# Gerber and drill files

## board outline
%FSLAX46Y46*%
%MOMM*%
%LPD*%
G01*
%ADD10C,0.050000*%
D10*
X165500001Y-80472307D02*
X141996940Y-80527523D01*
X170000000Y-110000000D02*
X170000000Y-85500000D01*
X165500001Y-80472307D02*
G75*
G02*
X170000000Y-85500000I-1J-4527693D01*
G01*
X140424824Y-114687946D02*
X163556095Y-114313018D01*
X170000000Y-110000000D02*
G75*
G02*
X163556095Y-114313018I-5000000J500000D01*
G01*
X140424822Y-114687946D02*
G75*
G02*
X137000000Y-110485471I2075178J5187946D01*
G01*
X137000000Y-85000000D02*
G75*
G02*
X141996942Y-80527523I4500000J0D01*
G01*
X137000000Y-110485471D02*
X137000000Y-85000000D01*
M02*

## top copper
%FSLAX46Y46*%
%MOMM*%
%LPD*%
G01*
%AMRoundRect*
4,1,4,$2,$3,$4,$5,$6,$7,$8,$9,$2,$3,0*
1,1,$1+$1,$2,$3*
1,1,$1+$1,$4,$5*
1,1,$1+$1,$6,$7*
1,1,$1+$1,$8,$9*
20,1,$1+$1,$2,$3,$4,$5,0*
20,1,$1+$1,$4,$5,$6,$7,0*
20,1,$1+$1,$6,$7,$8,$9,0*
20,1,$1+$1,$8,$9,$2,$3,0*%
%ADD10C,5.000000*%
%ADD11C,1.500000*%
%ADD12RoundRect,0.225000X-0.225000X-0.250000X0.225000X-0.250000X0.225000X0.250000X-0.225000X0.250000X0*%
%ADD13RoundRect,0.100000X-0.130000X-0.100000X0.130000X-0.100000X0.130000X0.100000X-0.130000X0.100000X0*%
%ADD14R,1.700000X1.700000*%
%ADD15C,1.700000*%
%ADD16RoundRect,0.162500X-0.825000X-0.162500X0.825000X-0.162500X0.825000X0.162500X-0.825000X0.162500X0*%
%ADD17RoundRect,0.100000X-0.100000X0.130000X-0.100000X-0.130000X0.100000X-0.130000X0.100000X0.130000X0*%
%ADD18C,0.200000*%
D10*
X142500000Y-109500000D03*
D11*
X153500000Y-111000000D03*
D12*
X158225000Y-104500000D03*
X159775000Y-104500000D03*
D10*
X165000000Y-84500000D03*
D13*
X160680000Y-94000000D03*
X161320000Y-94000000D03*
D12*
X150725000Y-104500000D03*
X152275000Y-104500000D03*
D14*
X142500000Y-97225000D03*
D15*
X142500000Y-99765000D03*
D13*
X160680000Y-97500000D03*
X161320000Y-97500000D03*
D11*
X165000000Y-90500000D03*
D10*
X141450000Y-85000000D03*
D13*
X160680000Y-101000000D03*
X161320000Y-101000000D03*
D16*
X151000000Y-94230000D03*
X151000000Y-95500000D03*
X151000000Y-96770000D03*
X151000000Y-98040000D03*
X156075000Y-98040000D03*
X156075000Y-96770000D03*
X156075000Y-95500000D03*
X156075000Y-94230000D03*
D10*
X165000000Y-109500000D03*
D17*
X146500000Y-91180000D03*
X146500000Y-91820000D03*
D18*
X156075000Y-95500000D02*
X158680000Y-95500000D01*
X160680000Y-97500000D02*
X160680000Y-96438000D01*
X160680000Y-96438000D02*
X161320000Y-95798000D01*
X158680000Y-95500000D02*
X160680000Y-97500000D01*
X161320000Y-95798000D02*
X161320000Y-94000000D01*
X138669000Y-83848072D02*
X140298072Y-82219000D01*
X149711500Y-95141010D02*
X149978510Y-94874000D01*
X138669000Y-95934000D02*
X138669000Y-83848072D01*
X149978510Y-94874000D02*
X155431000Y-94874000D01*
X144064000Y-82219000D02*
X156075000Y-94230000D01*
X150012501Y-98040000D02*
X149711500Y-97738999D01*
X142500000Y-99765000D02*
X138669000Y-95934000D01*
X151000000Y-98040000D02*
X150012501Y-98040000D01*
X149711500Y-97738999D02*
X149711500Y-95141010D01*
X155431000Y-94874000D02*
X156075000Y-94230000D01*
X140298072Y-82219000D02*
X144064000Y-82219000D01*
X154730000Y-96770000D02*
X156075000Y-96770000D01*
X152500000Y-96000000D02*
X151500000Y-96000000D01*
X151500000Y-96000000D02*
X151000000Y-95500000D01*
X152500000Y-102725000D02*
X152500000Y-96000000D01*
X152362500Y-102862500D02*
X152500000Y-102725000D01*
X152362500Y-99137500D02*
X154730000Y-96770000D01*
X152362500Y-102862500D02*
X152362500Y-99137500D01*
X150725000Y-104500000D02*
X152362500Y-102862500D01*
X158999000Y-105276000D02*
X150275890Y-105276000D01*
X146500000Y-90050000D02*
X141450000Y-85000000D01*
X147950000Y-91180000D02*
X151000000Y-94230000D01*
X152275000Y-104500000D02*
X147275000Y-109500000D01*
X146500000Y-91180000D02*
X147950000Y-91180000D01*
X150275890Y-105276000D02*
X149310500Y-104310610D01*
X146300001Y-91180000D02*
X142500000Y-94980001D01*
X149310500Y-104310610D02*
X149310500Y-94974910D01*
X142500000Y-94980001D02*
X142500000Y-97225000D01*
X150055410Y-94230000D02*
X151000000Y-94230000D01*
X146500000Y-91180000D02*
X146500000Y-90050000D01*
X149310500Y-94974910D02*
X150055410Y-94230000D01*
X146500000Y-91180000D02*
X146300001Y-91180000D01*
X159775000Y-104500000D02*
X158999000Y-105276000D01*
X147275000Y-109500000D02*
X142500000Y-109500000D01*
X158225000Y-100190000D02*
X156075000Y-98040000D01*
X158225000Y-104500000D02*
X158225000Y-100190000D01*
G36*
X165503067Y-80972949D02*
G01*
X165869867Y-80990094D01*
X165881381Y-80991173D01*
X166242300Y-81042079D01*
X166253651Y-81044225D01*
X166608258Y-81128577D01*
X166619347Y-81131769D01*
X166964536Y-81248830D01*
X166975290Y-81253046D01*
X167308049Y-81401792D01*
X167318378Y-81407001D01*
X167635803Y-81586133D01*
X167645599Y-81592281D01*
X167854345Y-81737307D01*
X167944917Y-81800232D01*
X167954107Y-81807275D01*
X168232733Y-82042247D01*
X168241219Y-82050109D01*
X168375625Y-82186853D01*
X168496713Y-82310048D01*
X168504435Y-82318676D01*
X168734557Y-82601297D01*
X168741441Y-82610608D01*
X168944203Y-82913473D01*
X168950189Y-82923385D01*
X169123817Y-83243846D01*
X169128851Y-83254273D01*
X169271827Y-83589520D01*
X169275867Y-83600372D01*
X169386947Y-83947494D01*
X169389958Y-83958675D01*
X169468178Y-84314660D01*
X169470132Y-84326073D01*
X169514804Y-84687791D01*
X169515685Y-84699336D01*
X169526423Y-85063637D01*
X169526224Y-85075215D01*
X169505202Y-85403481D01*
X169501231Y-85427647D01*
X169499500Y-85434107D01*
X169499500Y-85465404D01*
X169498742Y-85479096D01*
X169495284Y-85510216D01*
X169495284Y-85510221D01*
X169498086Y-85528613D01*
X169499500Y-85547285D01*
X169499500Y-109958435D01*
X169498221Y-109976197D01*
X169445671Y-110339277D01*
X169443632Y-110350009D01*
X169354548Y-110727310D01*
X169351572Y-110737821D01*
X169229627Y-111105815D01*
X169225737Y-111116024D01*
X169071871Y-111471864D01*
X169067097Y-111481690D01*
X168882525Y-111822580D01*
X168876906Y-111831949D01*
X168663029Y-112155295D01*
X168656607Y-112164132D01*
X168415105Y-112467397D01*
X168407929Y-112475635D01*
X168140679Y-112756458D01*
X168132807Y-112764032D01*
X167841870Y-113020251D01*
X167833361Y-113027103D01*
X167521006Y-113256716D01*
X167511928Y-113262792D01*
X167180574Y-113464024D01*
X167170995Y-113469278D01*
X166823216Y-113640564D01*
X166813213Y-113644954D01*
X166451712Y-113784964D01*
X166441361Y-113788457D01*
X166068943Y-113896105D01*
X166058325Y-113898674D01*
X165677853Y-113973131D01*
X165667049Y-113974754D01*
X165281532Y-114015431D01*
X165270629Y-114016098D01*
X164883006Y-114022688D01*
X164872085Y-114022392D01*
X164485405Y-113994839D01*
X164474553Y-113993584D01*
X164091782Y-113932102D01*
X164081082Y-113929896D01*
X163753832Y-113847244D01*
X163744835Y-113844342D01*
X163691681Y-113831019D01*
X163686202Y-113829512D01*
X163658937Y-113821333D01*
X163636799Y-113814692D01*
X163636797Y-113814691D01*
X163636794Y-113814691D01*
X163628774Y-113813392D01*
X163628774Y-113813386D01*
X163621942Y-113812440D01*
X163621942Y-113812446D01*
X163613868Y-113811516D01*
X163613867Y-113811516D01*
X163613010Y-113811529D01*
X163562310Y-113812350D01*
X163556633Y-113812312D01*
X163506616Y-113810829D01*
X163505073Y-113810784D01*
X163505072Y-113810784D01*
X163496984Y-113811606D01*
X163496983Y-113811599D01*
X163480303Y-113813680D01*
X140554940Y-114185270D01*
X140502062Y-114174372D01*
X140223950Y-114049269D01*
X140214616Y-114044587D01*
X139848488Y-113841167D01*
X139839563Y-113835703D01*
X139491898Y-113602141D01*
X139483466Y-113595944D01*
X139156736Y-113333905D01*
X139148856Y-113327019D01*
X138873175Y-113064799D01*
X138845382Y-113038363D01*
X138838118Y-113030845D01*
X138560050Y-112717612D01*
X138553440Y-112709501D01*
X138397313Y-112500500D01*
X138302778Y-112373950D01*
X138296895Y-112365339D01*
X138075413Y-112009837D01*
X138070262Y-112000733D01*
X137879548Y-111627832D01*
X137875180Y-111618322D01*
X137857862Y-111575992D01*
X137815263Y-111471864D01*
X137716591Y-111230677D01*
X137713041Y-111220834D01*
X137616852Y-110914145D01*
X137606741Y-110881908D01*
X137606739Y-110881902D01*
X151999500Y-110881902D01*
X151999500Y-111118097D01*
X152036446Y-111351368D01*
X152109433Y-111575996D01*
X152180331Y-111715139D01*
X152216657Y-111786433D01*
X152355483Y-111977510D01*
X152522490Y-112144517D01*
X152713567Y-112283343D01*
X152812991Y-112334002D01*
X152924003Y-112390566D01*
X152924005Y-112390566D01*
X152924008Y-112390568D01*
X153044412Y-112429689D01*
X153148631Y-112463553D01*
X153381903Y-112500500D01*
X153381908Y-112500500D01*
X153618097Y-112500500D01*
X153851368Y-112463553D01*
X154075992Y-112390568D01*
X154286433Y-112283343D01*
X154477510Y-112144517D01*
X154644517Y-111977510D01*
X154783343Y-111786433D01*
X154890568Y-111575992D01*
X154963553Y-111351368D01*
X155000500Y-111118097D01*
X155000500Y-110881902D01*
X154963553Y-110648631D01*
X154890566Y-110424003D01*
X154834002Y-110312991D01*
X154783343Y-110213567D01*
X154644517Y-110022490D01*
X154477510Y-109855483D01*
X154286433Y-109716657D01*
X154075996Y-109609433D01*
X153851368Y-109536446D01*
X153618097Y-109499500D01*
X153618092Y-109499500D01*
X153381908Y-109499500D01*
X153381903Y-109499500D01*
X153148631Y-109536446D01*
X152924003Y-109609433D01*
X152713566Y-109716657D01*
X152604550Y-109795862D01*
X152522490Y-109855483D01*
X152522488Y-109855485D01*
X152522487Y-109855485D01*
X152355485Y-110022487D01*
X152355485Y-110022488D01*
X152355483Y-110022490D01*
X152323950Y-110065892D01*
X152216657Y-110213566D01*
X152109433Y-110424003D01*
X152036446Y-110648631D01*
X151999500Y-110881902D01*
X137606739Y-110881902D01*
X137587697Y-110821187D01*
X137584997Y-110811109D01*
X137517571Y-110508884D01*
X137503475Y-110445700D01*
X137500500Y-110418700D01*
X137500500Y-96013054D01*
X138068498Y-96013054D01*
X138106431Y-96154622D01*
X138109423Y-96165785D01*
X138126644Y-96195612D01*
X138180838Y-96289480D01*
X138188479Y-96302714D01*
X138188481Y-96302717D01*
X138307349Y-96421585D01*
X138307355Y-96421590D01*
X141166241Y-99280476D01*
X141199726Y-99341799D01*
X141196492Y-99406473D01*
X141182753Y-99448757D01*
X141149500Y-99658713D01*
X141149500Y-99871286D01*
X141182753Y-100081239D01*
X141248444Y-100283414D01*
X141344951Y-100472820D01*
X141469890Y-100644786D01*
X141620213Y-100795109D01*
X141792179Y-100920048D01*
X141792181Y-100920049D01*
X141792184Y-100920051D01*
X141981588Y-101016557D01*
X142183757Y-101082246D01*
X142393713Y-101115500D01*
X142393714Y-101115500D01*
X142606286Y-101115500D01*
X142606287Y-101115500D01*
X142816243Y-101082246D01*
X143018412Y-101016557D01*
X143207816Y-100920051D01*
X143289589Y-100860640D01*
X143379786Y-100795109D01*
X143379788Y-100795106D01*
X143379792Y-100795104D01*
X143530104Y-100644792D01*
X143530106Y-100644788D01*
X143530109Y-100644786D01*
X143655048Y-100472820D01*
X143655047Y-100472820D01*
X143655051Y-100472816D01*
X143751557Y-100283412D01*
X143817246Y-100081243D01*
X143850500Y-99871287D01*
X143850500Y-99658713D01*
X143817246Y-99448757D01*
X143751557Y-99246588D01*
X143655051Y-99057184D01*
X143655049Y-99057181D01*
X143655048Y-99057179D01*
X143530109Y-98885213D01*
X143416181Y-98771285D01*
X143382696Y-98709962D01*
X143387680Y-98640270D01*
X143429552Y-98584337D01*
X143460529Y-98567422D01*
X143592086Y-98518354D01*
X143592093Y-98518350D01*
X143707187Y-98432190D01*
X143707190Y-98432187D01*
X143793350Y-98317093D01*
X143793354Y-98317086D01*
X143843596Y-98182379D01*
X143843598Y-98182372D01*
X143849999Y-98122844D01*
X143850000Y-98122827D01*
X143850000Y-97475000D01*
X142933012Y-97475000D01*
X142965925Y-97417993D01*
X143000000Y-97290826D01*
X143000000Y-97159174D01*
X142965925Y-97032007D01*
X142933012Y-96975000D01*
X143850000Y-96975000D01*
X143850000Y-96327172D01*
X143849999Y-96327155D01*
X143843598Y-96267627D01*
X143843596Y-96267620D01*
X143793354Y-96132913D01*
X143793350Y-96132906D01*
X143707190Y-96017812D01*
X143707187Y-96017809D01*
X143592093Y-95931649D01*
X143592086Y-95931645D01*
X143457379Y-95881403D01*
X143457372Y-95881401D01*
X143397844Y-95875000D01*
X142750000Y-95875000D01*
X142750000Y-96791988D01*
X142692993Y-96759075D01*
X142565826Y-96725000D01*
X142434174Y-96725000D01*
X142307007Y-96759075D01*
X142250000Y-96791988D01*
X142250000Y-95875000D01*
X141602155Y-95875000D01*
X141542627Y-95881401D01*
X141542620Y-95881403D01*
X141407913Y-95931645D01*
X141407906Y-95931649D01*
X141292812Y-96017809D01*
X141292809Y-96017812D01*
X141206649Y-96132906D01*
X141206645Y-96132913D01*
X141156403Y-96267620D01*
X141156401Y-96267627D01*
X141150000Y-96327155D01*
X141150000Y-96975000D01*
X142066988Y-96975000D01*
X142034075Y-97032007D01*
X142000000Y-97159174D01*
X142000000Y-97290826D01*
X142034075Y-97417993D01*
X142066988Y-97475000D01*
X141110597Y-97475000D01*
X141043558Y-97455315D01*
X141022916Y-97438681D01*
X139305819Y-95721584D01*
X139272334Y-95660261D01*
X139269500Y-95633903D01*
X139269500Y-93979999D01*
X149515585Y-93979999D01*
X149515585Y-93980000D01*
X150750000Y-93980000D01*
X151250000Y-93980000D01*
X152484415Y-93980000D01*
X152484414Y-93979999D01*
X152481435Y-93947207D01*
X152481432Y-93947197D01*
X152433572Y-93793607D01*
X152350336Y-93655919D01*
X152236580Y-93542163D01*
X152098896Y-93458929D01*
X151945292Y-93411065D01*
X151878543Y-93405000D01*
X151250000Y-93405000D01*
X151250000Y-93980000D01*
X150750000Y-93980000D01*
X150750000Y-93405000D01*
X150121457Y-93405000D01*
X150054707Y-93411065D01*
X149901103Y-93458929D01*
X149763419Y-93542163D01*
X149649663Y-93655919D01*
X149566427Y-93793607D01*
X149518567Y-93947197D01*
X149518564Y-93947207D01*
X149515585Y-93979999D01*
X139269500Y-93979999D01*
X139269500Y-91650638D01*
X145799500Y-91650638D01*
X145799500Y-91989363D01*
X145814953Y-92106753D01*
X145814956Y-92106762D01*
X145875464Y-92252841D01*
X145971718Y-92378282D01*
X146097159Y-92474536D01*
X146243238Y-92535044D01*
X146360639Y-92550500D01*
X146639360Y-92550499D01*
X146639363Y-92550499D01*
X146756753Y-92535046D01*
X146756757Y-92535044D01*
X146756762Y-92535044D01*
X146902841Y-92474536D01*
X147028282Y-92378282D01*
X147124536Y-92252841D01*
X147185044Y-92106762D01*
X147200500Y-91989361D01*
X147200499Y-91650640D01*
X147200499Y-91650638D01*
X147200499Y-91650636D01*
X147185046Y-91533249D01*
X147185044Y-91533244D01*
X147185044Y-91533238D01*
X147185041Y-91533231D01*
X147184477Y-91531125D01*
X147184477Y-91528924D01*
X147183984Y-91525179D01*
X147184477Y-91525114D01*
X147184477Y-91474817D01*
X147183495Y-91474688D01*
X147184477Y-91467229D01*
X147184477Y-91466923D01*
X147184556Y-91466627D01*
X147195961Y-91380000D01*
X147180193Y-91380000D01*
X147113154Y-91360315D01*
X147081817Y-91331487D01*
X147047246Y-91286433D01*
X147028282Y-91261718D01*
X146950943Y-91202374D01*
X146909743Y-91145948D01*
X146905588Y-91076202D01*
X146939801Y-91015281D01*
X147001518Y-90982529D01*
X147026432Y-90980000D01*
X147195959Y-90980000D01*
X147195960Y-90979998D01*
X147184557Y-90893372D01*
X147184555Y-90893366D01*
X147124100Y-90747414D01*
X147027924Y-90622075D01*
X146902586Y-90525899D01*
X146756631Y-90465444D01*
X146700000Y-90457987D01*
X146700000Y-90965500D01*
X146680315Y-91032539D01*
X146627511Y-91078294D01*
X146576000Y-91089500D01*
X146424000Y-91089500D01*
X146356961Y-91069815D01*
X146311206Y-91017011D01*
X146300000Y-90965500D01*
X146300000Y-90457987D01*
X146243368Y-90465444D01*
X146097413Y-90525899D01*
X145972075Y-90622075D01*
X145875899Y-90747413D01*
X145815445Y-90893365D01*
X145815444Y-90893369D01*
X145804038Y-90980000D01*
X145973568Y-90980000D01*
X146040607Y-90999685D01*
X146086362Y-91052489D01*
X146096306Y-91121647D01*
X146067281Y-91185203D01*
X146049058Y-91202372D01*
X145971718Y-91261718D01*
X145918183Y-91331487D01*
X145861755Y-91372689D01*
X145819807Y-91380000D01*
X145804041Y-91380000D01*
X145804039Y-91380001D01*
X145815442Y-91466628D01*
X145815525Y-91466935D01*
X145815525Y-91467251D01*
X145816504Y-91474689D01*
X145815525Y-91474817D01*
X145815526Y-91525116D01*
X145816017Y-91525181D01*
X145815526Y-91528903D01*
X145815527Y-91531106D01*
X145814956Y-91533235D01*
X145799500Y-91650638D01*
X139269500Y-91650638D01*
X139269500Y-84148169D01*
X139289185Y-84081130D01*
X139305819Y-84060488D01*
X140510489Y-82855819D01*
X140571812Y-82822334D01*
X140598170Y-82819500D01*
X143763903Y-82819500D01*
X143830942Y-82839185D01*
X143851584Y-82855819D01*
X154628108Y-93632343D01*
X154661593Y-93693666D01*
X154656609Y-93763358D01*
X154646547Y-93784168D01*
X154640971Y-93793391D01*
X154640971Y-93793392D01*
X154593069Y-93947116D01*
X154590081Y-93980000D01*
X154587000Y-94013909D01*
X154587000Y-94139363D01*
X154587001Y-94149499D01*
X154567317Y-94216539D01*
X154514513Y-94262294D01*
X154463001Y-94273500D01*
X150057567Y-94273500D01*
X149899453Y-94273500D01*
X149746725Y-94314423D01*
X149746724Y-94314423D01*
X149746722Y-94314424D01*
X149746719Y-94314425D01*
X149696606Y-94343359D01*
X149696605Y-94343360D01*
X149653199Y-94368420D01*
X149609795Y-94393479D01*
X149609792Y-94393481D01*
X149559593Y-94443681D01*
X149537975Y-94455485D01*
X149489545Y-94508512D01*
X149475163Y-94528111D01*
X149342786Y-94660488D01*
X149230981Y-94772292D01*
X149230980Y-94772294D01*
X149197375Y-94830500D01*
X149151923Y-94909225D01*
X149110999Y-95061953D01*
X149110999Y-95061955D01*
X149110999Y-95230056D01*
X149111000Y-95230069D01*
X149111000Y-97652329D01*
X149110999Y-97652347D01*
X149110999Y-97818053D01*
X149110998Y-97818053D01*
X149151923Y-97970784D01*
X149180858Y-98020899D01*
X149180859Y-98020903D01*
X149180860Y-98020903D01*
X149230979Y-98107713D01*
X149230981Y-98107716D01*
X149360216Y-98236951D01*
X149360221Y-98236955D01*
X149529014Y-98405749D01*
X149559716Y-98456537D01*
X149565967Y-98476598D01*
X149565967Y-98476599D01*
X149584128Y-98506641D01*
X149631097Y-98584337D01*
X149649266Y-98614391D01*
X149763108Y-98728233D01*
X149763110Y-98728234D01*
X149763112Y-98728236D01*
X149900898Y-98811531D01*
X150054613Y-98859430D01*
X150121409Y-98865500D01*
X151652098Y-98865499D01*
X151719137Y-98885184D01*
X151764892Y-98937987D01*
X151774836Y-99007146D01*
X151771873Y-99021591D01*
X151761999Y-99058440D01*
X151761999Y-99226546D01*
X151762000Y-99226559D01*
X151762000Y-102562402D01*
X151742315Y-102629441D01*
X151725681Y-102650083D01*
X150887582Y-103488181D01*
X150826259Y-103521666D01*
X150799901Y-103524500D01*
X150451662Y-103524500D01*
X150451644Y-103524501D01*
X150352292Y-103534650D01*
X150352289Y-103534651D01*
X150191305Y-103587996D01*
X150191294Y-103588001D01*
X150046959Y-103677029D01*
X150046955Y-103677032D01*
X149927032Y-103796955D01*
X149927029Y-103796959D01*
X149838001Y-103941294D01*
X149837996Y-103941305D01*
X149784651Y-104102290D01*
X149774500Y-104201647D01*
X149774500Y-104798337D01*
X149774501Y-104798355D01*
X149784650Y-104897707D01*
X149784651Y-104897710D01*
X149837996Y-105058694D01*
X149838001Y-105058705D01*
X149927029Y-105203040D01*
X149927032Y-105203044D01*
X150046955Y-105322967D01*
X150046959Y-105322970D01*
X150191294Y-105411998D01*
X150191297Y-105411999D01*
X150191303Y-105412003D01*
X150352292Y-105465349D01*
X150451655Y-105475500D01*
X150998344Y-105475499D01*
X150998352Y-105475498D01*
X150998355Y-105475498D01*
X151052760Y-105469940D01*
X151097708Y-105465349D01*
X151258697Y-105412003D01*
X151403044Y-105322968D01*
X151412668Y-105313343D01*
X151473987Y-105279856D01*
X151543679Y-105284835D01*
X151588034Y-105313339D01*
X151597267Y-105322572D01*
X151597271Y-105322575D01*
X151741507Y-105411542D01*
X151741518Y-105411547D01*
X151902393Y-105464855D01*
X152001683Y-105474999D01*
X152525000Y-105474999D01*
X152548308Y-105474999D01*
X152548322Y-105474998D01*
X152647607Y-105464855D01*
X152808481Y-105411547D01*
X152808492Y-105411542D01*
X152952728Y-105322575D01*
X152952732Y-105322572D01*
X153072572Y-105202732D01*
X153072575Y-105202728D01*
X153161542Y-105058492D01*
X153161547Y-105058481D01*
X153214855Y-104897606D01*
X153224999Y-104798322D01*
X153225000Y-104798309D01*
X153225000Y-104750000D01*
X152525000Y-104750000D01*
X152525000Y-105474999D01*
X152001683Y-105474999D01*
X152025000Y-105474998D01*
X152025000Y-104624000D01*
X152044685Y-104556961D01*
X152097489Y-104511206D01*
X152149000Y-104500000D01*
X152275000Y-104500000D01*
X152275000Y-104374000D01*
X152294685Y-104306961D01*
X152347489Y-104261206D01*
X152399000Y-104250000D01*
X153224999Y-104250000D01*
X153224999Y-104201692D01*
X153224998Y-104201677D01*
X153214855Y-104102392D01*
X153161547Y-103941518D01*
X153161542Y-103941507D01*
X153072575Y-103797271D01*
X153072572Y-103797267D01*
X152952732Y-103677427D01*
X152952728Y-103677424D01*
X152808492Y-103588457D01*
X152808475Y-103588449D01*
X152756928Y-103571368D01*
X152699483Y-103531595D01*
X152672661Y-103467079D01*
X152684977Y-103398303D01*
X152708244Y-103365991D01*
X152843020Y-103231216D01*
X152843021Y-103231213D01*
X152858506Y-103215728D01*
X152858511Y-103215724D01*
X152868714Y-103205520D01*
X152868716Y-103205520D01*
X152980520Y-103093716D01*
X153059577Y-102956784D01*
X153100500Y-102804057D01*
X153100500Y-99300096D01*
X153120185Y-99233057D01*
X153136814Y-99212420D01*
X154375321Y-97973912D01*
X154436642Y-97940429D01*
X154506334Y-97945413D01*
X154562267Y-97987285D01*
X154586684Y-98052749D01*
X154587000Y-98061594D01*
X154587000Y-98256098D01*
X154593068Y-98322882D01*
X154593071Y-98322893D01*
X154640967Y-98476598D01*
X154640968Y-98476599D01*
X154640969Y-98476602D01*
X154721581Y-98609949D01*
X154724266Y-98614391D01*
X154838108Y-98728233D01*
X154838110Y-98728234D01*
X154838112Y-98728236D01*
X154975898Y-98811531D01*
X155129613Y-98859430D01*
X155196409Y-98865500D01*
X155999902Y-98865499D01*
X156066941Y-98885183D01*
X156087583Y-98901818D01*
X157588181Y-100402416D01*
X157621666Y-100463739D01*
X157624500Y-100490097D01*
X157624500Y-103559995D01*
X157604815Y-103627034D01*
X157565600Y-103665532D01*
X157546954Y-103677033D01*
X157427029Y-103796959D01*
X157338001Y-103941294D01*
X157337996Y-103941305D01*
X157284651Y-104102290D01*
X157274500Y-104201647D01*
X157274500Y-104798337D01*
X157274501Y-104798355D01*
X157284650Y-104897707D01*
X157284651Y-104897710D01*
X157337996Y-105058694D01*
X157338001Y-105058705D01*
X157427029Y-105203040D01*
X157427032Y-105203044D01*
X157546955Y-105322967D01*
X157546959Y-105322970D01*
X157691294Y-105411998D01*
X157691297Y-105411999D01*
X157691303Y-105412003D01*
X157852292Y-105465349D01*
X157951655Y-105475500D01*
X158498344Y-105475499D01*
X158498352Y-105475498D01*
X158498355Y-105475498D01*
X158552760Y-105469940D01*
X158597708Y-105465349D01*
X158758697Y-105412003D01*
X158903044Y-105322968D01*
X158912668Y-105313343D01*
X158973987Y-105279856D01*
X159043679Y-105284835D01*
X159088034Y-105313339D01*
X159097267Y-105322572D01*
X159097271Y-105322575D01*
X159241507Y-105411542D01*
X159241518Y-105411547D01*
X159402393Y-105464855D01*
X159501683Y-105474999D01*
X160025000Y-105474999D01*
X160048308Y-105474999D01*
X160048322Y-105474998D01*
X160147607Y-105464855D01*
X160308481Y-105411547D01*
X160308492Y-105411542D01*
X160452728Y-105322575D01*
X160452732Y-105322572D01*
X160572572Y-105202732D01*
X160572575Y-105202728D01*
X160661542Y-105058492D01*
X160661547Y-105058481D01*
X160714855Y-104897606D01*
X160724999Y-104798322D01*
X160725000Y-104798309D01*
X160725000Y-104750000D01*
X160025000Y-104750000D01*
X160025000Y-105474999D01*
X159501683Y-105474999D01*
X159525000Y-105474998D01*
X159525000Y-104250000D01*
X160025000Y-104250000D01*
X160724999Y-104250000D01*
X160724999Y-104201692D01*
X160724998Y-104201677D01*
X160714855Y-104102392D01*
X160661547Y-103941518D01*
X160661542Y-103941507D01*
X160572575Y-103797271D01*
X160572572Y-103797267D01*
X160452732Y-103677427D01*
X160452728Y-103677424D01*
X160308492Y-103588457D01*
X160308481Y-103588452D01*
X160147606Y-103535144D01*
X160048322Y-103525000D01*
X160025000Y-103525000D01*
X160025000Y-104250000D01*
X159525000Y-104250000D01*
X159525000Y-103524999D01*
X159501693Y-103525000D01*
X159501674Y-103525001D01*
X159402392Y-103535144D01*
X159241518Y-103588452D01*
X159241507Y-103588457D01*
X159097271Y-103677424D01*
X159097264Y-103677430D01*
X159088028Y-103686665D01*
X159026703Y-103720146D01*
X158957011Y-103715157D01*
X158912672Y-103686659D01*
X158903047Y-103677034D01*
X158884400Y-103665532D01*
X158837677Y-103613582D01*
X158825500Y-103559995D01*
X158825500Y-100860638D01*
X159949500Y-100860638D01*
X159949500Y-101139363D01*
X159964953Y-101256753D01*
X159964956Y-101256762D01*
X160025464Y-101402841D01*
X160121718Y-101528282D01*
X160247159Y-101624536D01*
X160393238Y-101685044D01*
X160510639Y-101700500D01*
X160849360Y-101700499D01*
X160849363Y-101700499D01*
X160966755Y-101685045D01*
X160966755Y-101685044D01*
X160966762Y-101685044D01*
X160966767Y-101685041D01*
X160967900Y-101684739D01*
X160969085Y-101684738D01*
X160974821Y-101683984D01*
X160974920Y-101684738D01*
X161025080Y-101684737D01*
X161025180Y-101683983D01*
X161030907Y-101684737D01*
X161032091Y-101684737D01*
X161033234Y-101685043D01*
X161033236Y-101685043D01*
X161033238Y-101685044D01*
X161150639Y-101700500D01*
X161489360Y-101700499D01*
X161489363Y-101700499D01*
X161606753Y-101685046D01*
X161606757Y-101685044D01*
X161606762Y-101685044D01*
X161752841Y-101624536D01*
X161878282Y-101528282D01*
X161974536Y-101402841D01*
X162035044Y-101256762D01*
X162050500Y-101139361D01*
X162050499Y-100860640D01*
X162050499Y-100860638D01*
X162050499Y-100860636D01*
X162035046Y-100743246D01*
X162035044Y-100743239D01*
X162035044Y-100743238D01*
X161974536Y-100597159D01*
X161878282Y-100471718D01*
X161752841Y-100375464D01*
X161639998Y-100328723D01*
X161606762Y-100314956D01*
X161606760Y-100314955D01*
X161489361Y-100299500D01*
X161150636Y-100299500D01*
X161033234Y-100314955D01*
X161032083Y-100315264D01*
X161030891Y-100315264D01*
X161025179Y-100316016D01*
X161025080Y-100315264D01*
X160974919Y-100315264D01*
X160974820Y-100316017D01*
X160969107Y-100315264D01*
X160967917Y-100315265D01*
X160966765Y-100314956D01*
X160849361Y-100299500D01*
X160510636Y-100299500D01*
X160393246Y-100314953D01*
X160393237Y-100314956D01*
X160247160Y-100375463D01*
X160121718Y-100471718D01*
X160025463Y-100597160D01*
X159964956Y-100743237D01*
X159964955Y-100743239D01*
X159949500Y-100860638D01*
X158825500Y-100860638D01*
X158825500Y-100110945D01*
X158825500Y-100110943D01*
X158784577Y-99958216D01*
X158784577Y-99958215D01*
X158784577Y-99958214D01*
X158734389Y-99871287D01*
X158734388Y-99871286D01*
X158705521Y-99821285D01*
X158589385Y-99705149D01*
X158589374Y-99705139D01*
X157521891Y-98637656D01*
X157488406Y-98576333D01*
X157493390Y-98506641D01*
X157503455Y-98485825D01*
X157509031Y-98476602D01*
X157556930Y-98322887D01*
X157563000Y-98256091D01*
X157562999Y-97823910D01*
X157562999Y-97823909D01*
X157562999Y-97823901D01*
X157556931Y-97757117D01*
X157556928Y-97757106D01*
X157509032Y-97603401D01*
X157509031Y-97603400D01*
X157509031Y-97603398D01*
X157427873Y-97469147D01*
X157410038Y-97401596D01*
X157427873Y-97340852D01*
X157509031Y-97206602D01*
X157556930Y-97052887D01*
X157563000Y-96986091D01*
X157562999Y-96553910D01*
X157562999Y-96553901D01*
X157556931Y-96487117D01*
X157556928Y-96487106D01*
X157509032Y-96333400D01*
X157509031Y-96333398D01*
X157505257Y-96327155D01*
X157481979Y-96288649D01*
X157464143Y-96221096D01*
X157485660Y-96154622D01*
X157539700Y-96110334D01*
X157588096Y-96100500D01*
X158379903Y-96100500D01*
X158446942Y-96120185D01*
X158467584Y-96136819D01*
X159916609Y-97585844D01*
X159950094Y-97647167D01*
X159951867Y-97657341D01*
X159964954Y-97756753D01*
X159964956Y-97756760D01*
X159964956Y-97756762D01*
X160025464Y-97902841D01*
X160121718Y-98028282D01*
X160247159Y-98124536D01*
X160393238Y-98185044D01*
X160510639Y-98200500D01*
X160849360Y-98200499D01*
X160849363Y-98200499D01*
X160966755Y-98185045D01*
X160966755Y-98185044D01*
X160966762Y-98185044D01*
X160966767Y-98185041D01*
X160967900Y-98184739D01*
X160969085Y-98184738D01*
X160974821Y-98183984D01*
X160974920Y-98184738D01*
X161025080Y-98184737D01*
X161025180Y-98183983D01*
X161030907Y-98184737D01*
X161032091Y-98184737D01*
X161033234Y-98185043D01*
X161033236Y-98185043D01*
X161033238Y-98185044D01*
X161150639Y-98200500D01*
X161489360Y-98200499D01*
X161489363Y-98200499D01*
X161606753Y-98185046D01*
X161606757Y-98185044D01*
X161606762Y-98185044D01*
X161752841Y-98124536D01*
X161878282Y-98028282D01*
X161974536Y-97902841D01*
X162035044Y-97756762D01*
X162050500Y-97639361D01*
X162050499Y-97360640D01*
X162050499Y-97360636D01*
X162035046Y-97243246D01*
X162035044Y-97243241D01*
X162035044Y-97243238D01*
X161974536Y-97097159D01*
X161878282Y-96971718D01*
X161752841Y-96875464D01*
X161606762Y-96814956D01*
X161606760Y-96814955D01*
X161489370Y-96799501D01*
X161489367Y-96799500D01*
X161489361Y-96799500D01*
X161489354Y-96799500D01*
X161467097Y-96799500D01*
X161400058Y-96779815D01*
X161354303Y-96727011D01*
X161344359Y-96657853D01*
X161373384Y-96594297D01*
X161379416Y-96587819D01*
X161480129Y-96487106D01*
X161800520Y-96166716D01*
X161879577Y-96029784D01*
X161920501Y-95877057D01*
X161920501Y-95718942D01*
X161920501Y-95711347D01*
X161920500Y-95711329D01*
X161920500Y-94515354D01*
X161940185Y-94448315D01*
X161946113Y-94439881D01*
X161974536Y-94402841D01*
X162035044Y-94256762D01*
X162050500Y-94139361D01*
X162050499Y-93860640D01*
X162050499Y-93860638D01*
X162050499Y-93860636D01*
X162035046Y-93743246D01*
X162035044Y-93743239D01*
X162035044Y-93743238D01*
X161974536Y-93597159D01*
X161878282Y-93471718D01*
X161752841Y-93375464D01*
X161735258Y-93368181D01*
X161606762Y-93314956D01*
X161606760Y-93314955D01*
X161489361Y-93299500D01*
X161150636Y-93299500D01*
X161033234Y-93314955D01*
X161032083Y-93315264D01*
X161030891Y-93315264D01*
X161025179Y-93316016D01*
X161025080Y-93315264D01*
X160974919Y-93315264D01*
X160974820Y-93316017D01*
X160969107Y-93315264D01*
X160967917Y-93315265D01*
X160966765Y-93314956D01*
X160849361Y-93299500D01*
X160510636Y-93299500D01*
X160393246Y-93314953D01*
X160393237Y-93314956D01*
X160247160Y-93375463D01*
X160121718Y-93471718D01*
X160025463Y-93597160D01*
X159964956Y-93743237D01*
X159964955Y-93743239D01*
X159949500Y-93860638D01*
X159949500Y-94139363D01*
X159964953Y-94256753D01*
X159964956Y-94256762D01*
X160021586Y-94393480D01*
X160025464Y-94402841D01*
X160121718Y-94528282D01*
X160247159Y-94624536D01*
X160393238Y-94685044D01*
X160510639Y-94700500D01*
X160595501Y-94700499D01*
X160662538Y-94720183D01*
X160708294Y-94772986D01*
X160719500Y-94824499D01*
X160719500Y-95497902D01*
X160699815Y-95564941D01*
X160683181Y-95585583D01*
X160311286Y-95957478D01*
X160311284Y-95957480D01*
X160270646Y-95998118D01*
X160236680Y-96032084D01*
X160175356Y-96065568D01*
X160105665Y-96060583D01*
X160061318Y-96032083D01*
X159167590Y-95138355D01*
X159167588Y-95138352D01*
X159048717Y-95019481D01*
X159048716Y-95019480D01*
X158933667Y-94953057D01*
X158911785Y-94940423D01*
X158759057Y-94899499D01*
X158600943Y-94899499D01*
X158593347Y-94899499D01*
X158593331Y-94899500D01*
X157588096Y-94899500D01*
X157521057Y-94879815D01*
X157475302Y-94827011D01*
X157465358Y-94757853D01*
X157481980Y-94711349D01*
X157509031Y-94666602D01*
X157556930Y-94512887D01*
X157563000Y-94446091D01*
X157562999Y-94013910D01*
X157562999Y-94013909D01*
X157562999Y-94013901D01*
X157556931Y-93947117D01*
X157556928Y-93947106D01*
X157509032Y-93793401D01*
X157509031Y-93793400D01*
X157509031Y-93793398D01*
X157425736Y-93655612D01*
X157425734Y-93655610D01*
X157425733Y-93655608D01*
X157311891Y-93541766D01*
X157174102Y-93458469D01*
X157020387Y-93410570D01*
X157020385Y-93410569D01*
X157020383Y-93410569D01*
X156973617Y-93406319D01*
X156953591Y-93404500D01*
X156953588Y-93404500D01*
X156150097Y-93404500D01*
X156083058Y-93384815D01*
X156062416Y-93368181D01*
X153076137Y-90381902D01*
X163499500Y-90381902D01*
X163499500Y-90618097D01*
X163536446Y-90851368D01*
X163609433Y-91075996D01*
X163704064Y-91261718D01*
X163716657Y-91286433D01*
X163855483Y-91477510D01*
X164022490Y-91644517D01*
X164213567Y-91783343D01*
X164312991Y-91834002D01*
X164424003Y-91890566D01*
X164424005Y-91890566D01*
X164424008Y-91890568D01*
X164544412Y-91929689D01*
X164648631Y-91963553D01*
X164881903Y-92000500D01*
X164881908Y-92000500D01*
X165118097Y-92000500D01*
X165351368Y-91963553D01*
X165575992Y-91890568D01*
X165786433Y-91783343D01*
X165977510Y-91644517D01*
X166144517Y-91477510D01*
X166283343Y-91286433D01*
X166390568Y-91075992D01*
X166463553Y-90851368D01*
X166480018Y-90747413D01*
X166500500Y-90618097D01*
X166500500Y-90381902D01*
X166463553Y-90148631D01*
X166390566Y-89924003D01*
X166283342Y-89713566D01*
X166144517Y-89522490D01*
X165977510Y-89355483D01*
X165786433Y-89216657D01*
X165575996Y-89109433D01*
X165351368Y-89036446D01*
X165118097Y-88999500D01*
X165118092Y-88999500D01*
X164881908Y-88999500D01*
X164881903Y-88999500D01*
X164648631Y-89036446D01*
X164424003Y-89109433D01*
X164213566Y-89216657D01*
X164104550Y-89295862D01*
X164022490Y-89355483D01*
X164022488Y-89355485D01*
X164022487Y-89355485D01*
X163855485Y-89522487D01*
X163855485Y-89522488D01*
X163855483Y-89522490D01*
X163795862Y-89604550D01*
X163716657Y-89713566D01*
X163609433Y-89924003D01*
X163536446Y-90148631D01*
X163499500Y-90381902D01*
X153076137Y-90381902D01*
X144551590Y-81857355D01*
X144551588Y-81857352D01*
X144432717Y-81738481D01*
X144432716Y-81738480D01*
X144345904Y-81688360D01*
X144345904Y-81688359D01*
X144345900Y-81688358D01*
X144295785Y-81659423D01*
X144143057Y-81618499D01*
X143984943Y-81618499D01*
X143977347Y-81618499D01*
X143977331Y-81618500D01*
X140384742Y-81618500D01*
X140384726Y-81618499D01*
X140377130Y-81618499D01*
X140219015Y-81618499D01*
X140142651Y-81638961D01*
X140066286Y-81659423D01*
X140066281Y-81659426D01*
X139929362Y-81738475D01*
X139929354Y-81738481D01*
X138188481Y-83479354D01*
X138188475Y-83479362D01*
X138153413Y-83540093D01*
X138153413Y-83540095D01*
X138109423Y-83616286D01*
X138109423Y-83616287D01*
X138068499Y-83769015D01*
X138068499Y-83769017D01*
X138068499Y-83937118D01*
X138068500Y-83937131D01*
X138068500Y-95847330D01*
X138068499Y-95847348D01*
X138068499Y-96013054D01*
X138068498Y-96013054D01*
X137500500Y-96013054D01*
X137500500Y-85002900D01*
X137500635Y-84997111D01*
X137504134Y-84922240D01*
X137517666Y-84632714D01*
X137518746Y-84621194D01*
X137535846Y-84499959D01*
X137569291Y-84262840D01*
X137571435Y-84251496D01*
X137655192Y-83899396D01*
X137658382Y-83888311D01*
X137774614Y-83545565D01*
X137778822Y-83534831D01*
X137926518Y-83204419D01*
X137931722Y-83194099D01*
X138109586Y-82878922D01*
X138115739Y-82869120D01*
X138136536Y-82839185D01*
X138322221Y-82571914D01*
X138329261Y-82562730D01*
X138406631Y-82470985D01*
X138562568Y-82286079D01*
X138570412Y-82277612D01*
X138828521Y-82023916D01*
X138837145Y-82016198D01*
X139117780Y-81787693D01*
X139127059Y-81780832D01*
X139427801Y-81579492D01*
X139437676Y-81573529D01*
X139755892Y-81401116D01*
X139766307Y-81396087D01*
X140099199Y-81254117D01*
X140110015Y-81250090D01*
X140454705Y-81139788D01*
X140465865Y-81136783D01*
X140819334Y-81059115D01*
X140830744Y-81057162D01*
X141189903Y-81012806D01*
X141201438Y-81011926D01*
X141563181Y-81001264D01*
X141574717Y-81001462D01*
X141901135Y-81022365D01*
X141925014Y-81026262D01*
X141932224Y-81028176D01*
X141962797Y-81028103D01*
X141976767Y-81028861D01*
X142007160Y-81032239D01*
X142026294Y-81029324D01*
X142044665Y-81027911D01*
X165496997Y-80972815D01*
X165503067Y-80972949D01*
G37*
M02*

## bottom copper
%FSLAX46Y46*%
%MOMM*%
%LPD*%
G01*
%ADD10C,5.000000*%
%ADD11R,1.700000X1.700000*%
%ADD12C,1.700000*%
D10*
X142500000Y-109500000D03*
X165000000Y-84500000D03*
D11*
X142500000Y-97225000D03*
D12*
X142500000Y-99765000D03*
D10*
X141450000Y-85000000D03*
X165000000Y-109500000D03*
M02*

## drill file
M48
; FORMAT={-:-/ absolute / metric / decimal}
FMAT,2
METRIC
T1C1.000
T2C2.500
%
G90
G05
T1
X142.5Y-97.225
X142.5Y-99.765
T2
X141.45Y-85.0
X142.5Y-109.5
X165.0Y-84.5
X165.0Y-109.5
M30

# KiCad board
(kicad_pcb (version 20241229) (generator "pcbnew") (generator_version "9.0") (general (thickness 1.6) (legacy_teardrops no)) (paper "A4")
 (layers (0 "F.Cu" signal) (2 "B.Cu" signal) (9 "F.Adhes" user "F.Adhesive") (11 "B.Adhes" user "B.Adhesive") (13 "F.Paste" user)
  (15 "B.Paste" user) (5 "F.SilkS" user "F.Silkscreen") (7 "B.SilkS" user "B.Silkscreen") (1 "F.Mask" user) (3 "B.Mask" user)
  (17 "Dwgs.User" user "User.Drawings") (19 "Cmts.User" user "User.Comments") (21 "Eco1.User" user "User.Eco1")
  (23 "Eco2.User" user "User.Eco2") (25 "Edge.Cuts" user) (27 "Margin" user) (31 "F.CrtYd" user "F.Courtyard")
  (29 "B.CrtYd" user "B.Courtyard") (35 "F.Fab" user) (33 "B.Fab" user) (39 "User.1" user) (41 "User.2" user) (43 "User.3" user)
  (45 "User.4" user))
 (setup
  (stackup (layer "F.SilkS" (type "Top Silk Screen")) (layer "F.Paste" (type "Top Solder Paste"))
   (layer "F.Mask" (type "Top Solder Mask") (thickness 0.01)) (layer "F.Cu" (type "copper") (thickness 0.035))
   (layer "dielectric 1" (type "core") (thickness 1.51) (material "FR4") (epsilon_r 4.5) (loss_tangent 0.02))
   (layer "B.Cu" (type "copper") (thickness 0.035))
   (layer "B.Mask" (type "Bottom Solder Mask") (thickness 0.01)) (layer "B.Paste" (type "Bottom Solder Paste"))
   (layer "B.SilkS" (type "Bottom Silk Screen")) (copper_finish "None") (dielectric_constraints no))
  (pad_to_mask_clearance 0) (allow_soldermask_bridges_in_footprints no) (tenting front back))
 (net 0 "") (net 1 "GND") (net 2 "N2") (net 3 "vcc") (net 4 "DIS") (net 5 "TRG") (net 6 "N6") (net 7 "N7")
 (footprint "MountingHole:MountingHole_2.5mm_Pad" (layer "F.Cu") (at 142.5 109.5)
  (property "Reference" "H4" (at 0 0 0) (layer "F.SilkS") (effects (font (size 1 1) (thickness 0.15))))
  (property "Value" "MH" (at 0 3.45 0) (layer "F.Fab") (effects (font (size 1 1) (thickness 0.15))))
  (pad "1" thru_hole circle (at 0 0) (size 5 5) (drill 2.5) (layers "*.Cu" "*.Mask") (remove_unused_layers no) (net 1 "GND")
   (zone_connect 2)))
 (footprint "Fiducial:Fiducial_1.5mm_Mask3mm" (layer "F.Cu") (at 153.5 111)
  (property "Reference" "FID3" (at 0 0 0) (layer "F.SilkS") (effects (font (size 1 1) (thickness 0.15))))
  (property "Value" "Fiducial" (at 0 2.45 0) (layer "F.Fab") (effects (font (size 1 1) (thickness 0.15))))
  (pad "" smd circle (at 0 0) (size 1.5 1.5) (layers "F.Cu" "F.Mask") (solder_mask_margin 0.75) (clearance 0.75)))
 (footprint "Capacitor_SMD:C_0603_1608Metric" (layer "F.Cu") (at 159 104.5)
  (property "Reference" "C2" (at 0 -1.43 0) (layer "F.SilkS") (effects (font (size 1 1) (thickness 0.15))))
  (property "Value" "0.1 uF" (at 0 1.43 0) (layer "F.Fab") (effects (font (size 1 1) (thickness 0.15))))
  (pad "1" smd roundrect (at -0.775 0) (size 0.9 0.95) (layers "F.Cu" "F.Mask" "F.Paste") (roundrect_rratio 0.25) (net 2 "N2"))
  (pad "2" smd roundrect (at 0.775 0) (size 0.9 0.95) (layers "F.Cu" "F.Mask" "F.Paste") (roundrect_rratio 0.25) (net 1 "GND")))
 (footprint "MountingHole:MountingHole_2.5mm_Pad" (layer "F.Cu") (at 165 84.5)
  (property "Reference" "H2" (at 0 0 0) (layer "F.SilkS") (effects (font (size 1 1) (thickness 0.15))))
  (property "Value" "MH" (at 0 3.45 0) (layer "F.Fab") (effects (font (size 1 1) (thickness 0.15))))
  (pad "1" thru_hole circle (at 0 0) (size 5 5) (drill 2.5) (layers "*.Cu" "*.Mask") (remove_unused_layers no) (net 1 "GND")
   (zone_connect 2)))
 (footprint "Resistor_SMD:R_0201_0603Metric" (layer "F.Cu") (at 161 94)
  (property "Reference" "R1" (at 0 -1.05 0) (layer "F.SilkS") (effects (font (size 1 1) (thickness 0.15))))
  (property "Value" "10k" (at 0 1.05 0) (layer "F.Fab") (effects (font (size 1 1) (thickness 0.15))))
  (pad "" smd roundrect (at -0.345 0) (size 0.318 0.36) (layers "F.Paste") (roundrect_rratio 0.25))
  (pad "" smd roundrect (at 0.345 0) (size 0.318 0.36) (layers "F.Paste") (roundrect_rratio 0.25))
  (pad "1" smd roundrect (at -0.32 0) (size 0.46 0.4) (layers "F.Cu" "F.Mask") (roundrect_rratio 0.25) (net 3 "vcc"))
  (pad "2" smd roundrect (at 0.32 0) (size 0.46 0.4) (layers "F.Cu" "F.Mask") (roundrect_rratio 0.25) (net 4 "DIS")))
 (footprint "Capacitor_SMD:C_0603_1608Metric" (layer "F.Cu") (at 151.5 104.5)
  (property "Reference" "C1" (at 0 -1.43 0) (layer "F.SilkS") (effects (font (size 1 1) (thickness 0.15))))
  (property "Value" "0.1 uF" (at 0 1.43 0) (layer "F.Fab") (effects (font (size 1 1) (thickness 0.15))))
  (pad "1" smd roundrect (at -0.775 0) (size 0.9 0.95) (layers "F.Cu" "F.Mask" "F.Paste") (roundrect_rratio 0.25) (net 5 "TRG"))
  (pad "2" smd roundrect (at 0.775 0) (size 0.9 0.95) (layers "F.Cu" "F.Mask" "F.Paste") (roundrect_rratio 0.25) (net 1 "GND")))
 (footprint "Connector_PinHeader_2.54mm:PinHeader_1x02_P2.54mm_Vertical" (layer "F.Cu") (at 142.5 97.225)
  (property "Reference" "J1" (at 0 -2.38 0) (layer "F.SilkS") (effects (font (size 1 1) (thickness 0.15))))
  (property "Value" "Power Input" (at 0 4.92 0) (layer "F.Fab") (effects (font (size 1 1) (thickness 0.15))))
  (pad "1" thru_hole rect (at 0 0) (size 1.7 1.7) (drill 1) (layers "*.Cu" "*.Mask") (remove_unused_layers no) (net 1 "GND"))
  (pad "2" thru_hole circle (at 0 2.54) (size 1.7 1.7) (drill 1) (layers "*.Cu" "*.Mask") (remove_unused_layers no) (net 3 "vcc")))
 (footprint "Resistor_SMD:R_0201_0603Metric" (layer "F.Cu") (at 161 97.5)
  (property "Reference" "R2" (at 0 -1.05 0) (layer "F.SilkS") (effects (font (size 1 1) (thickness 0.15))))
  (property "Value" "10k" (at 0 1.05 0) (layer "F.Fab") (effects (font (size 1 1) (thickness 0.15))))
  (pad "" smd roundrect (at -0.345 0) (size 0.318 0.36) (layers "F.Paste") (roundrect_rratio 0.25))
  (pad "" smd roundrect (at 0.345 0) (size 0.318 0.36) (layers "F.Paste") (roundrect_rratio 0.25))
  (pad "1" smd roundrect (at -0.32 0) (size 0.46 0.4) (layers "F.Cu" "F.Mask") (roundrect_rratio 0.25) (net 4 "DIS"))
  (pad "2" smd roundrect (at 0.32 0) (size 0.46 0.4) (layers "F.Cu" "F.Mask") (roundrect_rratio 0.25) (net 5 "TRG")))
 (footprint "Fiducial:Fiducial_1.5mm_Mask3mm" (layer "F.Cu") (at 165 90.5)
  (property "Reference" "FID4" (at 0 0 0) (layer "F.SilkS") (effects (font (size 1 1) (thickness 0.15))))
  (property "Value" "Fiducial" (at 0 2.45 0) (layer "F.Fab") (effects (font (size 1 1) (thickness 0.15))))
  (pad "" smd circle (at 0 0) (size 1.5 1.5) (layers "F.Cu" "F.Mask") (solder_mask_margin 0.75) (clearance 0.75)))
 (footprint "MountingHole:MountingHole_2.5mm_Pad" (layer "F.Cu") (at 141.45 85)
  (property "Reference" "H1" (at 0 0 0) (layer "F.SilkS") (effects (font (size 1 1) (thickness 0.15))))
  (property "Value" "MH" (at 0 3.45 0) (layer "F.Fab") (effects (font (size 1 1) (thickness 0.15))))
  (pad "1" thru_hole circle (at 0 0) (size 5 5) (drill 2.5) (layers "*.Cu" "*.Mask") (remove_unused_layers no) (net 1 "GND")
   (zone_connect 2)))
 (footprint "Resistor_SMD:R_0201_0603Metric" (layer "F.Cu") (at 161 101)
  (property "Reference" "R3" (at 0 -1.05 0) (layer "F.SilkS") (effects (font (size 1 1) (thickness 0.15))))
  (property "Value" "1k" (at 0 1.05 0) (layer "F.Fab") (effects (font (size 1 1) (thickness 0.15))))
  (pad "" smd roundrect (at -0.345 0) (size 0.318 0.36) (layers "F.Paste") (roundrect_rratio 0.25))
  (pad "" smd roundrect (at 0.345 0) (size 0.318 0.36) (layers "F.Paste") (roundrect_rratio 0.25))
  (pad "1" smd roundrect (at -0.32 0) (size 0.46 0.4) (layers "F.Cu" "F.Mask") (roundrect_rratio 0.25) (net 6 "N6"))
  (pad "2" smd roundrect (at 0.32 0) (size 0.46 0.4) (layers "F.Cu" "F.Mask") (roundrect_rratio 0.25) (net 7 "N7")))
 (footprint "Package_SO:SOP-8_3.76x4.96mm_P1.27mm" (layer "F.Cu") (at 153.5375 96.135)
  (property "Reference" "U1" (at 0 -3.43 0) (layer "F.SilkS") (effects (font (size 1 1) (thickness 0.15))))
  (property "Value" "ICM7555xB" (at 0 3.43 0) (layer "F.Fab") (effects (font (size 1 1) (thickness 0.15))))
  (pad "1" smd roundrect (at -2.5375 -1.905) (size 1.975 0.65) (layers "F.Cu" "F.Mask" "F.Paste") (roundrect_rratio 0.25) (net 1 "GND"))
  (pad "2" smd roundrect (at -2.5375 -0.635) (size 1.975 0.65) (layers "F.Cu" "F.Mask" "F.Paste") (roundrect_rratio 0.25) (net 5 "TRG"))
  (pad "3" smd roundrect (at -2.5375 0.635) (size 1.975 0.65) (layers "F.Cu" "F.Mask" "F.Paste") (roundrect_rratio 0.25) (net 6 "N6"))
  (pad "4" smd roundrect (at -2.5375 1.905) (size 1.975 0.65) (layers "F.Cu" "F.Mask" "F.Paste") (roundrect_rratio 0.25) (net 3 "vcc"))
  (pad "5" smd roundrect (at 2.5375 1.905) (size 1.975 0.65) (layers "F.Cu" "F.Mask" "F.Paste") (roundrect_rratio 0.25) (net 2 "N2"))
  (pad "6" smd roundrect (at 2.5375 0.635) (size 1.975 0.65) (layers "F.Cu" "F.Mask" "F.Paste") (roundrect_rratio 0.25) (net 5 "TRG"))
  (pad "7" smd roundrect (at 2.5375 -0.635) (size 1.975 0.65) (layers "F.Cu" "F.Mask" "F.Paste") (roundrect_rratio 0.25) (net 4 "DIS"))
  (pad "8" smd roundrect (at 2.5375 -1.905) (size 1.975 0.65) (layers "F.Cu" "F.Mask" "F.Paste") (roundrect_rratio 0.25) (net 3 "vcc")))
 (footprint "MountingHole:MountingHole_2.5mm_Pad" (layer "F.Cu") (at 165 109.5)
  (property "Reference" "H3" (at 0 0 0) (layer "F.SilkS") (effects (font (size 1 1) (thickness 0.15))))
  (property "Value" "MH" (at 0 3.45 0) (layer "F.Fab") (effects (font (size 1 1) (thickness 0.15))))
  (pad "1" thru_hole circle (at 0 0) (size 5 5) (drill 2.5) (layers "*.Cu" "*.Mask") (remove_unused_layers no) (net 1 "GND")
   (zone_connect 2)))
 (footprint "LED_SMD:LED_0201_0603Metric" (layer "F.Cu") (at 146.5 91.5 -90)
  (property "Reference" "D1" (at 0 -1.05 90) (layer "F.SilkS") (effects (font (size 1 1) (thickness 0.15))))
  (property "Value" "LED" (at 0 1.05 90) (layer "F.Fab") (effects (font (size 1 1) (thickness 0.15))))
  (pad "" smd roundrect (at -0.345 0 270) (size 0.318 0.36) (layers "F.Paste") (roundrect_rratio 0.25))
  (pad "" smd roundrect (at 0.345 0 270) (size 0.318 0.36) (layers "F.Paste") (roundrect_rratio 0.25))
  (pad "1" smd roundrect (at -0.32 0 270) (size 0.46 0.4) (layers "F.Cu" "F.Mask") (roundrect_rratio 0.25) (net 1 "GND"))
  (pad "2" smd roundrect (at 0.32 0 270) (size 0.46 0.4) (layers "F.Cu" "F.Mask") (roundrect_rratio 0.25) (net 7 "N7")))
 (gr_line (start 165.500001 80.472307) (end 141.99694 80.527523) (stroke (width 0.05) (type default)) (layer "Edge.Cuts"))
 (gr_line (start 170 110) (end 170 85.5) (stroke (width 0.05) (type default)) (layer "Edge.Cuts"))
 (gr_arc (start 165.500001 80.472307) (mid 168.873711 81.980385) (end 170 85.5) (stroke (width 0.05) (type default)) (layer "Edge.Cuts"))
 (gr_line (start 140.424824 114.687946) (end 163.556095 114.313018) (stroke (width 0.05) (type default)) (layer "Edge.Cuts"))
 (gr_arc (start 170 110) (mid 167.794993 113.675885) (end 163.556095 114.313018) (stroke (width 0.05) (type default)) (layer "Edge.Cuts"))
 (gr_arc (start 140.424822 114.687946) (mid 138.1686 113.029889) (end 137 110.485471) (stroke (width 0.05) (type default))
  (layer "Edge.Cuts"))
 (gr_arc (start 137 85) (mid 138.498853 81.646924) (end 141.996942 80.527523) (stroke (width 0.05) (type default)) (layer "Edge.Cuts"))
 (gr_line (start 137 110.485471) (end 137 85) (stroke (width 0.05) (type default)) (layer "Edge.Cuts"))
 (segment (start 156.075 95.5) (end 158.68 95.5) (width 0.2) (layer "F.Cu") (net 4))
 (segment (start 160.68 97.5) (end 160.68 96.438) (width 0.2) (layer "F.Cu") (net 4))
 (segment (start 160.68 96.438) (end 161.32 95.798) (width 0.2) (layer "F.Cu") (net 4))
 (segment (start 158.68 95.5) (end 160.68 97.5) (width 0.2) (layer "F.Cu") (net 4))
 (segment (start 161.32 95.798) (end 161.32 94) (width 0.2) (layer "F.Cu") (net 4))
 (segment (start 138.669 83.848072) (end 140.298072 82.219) (width 0.2) (layer "F.Cu") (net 3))
 (segment (start 149.7115 95.14101) (end 149.97851 94.874) (width 0.2) (layer "F.Cu") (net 3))
 (segment (start 138.669 95.934) (end 138.669 83.848072) (width 0.2) (layer "F.Cu") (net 3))
 (segment (start 149.97851 94.874) (end 155.431 94.874) (width 0.2) (layer "F.Cu") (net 3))
 (segment (start 144.064 82.219) (end 156.075 94.23) (width 0.2) (layer "F.Cu") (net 3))
 (segment (start 150.012501 98.04) (end 149.7115 97.738999) (width 0.2) (layer "F.Cu") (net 3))
 (segment (start 142.5 99.765) (end 138.669 95.934) (width 0.2) (layer "F.Cu") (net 3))
 (segment (start 151 98.04) (end 150.012501 98.04) (width 0.2) (layer "F.Cu") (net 3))
 (segment (start 149.7115 97.738999) (end 149.7115 95.14101) (width 0.2) (layer "F.Cu") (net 3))
 (segment (start 155.431 94.874) (end 156.075 94.23) (width 0.2) (layer "F.Cu") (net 3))
 (segment (start 140.298072 82.219) (end 144.064 82.219) (width 0.2) (layer "F.Cu") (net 3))
 (segment (start 154.73 96.77) (end 156.075 96.77) (width 0.2) (layer "F.Cu") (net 5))
 (segment (start 152.5 96) (end 151.5 96) (width 0.2) (layer "F.Cu") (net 5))
 (segment (start 151.5 96) (end 151 95.5) (width 0.2) (layer "F.Cu") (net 5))
 (segment (start 152.5 102.725) (end 152.5 96) (width 0.2) (layer "F.Cu") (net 5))
 (segment (start 152.3625 102.8625) (end 152.5 102.725) (width 0.2) (layer "F.Cu") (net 5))
 (segment (start 152.3625 99.1375) (end 154.73 96.77) (width 0.2) (layer "F.Cu") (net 5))
 (segment (start 152.3625 102.8625) (end 152.3625 99.1375) (width 0.2) (layer "F.Cu") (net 5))
 (segment (start 150.725 104.5) (end 152.3625 102.8625) (width 0.2) (layer "F.Cu") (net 5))
 (segment (start 158.999 105.276) (end 150.27589 105.276) (width 0.2) (layer "F.Cu") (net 1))
 (segment (start 146.5 90.05) (end 141.45 85) (width 0.2) (layer "F.Cu") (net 1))
 (segment (start 147.95 91.18) (end 151 94.23) (width 0.2) (layer "F.Cu") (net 1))
 (segment (start 152.275 104.5) (end 147.275 109.5) (width 0.2) (layer "F.Cu") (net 1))
 (segment (start 146.5 91.18) (end 147.95 91.18) (width 0.2) (layer "F.Cu") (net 1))
 (segment (start 150.27589 105.276) (end 149.3105 104.31061) (width 0.2) (layer "F.Cu") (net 1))
 (segment (start 146.300001 91.18) (end 142.5 94.980001) (width 0.2) (layer "F.Cu") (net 1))
 (segment (start 149.3105 104.31061) (end 149.3105 94.97491) (width 0.2) (layer "F.Cu") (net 1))
 (segment (start 142.5 94.980001) (end 142.5 97.225) (width 0.2) (layer "F.Cu") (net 1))
 (segment (start 150.05541 94.23) (end 151 94.23) (width 0.2) (layer "F.Cu") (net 1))
 (segment (start 146.5 91.18) (end 146.5 90.05) (width 0.2) (layer "F.Cu") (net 1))
 (segment (start 149.3105 94.97491) (end 150.05541 94.23) (width 0.2) (layer "F.Cu") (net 1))
 (segment (start 146.5 91.18) (end 146.300001 91.18) (width 0.2) (layer "F.Cu") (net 1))
 (segment (start 159.775 104.5) (end 158.999 105.276) (width 0.2) (layer "F.Cu") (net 1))
 (segment (start 147.275 109.5) (end 142.5 109.5) (width 0.2) (layer "F.Cu") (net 1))
 (segment (start 158.225 100.19) (end 156.075 98.04) (width 0.2) (layer "F.Cu") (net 2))
 (segment (start 158.225 104.5) (end 158.225 100.19) (width 0.2) (layer "F.Cu") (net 2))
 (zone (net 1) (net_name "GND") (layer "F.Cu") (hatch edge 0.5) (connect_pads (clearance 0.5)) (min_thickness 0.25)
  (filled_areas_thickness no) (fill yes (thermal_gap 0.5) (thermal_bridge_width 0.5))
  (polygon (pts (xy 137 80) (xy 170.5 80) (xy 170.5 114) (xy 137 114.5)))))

